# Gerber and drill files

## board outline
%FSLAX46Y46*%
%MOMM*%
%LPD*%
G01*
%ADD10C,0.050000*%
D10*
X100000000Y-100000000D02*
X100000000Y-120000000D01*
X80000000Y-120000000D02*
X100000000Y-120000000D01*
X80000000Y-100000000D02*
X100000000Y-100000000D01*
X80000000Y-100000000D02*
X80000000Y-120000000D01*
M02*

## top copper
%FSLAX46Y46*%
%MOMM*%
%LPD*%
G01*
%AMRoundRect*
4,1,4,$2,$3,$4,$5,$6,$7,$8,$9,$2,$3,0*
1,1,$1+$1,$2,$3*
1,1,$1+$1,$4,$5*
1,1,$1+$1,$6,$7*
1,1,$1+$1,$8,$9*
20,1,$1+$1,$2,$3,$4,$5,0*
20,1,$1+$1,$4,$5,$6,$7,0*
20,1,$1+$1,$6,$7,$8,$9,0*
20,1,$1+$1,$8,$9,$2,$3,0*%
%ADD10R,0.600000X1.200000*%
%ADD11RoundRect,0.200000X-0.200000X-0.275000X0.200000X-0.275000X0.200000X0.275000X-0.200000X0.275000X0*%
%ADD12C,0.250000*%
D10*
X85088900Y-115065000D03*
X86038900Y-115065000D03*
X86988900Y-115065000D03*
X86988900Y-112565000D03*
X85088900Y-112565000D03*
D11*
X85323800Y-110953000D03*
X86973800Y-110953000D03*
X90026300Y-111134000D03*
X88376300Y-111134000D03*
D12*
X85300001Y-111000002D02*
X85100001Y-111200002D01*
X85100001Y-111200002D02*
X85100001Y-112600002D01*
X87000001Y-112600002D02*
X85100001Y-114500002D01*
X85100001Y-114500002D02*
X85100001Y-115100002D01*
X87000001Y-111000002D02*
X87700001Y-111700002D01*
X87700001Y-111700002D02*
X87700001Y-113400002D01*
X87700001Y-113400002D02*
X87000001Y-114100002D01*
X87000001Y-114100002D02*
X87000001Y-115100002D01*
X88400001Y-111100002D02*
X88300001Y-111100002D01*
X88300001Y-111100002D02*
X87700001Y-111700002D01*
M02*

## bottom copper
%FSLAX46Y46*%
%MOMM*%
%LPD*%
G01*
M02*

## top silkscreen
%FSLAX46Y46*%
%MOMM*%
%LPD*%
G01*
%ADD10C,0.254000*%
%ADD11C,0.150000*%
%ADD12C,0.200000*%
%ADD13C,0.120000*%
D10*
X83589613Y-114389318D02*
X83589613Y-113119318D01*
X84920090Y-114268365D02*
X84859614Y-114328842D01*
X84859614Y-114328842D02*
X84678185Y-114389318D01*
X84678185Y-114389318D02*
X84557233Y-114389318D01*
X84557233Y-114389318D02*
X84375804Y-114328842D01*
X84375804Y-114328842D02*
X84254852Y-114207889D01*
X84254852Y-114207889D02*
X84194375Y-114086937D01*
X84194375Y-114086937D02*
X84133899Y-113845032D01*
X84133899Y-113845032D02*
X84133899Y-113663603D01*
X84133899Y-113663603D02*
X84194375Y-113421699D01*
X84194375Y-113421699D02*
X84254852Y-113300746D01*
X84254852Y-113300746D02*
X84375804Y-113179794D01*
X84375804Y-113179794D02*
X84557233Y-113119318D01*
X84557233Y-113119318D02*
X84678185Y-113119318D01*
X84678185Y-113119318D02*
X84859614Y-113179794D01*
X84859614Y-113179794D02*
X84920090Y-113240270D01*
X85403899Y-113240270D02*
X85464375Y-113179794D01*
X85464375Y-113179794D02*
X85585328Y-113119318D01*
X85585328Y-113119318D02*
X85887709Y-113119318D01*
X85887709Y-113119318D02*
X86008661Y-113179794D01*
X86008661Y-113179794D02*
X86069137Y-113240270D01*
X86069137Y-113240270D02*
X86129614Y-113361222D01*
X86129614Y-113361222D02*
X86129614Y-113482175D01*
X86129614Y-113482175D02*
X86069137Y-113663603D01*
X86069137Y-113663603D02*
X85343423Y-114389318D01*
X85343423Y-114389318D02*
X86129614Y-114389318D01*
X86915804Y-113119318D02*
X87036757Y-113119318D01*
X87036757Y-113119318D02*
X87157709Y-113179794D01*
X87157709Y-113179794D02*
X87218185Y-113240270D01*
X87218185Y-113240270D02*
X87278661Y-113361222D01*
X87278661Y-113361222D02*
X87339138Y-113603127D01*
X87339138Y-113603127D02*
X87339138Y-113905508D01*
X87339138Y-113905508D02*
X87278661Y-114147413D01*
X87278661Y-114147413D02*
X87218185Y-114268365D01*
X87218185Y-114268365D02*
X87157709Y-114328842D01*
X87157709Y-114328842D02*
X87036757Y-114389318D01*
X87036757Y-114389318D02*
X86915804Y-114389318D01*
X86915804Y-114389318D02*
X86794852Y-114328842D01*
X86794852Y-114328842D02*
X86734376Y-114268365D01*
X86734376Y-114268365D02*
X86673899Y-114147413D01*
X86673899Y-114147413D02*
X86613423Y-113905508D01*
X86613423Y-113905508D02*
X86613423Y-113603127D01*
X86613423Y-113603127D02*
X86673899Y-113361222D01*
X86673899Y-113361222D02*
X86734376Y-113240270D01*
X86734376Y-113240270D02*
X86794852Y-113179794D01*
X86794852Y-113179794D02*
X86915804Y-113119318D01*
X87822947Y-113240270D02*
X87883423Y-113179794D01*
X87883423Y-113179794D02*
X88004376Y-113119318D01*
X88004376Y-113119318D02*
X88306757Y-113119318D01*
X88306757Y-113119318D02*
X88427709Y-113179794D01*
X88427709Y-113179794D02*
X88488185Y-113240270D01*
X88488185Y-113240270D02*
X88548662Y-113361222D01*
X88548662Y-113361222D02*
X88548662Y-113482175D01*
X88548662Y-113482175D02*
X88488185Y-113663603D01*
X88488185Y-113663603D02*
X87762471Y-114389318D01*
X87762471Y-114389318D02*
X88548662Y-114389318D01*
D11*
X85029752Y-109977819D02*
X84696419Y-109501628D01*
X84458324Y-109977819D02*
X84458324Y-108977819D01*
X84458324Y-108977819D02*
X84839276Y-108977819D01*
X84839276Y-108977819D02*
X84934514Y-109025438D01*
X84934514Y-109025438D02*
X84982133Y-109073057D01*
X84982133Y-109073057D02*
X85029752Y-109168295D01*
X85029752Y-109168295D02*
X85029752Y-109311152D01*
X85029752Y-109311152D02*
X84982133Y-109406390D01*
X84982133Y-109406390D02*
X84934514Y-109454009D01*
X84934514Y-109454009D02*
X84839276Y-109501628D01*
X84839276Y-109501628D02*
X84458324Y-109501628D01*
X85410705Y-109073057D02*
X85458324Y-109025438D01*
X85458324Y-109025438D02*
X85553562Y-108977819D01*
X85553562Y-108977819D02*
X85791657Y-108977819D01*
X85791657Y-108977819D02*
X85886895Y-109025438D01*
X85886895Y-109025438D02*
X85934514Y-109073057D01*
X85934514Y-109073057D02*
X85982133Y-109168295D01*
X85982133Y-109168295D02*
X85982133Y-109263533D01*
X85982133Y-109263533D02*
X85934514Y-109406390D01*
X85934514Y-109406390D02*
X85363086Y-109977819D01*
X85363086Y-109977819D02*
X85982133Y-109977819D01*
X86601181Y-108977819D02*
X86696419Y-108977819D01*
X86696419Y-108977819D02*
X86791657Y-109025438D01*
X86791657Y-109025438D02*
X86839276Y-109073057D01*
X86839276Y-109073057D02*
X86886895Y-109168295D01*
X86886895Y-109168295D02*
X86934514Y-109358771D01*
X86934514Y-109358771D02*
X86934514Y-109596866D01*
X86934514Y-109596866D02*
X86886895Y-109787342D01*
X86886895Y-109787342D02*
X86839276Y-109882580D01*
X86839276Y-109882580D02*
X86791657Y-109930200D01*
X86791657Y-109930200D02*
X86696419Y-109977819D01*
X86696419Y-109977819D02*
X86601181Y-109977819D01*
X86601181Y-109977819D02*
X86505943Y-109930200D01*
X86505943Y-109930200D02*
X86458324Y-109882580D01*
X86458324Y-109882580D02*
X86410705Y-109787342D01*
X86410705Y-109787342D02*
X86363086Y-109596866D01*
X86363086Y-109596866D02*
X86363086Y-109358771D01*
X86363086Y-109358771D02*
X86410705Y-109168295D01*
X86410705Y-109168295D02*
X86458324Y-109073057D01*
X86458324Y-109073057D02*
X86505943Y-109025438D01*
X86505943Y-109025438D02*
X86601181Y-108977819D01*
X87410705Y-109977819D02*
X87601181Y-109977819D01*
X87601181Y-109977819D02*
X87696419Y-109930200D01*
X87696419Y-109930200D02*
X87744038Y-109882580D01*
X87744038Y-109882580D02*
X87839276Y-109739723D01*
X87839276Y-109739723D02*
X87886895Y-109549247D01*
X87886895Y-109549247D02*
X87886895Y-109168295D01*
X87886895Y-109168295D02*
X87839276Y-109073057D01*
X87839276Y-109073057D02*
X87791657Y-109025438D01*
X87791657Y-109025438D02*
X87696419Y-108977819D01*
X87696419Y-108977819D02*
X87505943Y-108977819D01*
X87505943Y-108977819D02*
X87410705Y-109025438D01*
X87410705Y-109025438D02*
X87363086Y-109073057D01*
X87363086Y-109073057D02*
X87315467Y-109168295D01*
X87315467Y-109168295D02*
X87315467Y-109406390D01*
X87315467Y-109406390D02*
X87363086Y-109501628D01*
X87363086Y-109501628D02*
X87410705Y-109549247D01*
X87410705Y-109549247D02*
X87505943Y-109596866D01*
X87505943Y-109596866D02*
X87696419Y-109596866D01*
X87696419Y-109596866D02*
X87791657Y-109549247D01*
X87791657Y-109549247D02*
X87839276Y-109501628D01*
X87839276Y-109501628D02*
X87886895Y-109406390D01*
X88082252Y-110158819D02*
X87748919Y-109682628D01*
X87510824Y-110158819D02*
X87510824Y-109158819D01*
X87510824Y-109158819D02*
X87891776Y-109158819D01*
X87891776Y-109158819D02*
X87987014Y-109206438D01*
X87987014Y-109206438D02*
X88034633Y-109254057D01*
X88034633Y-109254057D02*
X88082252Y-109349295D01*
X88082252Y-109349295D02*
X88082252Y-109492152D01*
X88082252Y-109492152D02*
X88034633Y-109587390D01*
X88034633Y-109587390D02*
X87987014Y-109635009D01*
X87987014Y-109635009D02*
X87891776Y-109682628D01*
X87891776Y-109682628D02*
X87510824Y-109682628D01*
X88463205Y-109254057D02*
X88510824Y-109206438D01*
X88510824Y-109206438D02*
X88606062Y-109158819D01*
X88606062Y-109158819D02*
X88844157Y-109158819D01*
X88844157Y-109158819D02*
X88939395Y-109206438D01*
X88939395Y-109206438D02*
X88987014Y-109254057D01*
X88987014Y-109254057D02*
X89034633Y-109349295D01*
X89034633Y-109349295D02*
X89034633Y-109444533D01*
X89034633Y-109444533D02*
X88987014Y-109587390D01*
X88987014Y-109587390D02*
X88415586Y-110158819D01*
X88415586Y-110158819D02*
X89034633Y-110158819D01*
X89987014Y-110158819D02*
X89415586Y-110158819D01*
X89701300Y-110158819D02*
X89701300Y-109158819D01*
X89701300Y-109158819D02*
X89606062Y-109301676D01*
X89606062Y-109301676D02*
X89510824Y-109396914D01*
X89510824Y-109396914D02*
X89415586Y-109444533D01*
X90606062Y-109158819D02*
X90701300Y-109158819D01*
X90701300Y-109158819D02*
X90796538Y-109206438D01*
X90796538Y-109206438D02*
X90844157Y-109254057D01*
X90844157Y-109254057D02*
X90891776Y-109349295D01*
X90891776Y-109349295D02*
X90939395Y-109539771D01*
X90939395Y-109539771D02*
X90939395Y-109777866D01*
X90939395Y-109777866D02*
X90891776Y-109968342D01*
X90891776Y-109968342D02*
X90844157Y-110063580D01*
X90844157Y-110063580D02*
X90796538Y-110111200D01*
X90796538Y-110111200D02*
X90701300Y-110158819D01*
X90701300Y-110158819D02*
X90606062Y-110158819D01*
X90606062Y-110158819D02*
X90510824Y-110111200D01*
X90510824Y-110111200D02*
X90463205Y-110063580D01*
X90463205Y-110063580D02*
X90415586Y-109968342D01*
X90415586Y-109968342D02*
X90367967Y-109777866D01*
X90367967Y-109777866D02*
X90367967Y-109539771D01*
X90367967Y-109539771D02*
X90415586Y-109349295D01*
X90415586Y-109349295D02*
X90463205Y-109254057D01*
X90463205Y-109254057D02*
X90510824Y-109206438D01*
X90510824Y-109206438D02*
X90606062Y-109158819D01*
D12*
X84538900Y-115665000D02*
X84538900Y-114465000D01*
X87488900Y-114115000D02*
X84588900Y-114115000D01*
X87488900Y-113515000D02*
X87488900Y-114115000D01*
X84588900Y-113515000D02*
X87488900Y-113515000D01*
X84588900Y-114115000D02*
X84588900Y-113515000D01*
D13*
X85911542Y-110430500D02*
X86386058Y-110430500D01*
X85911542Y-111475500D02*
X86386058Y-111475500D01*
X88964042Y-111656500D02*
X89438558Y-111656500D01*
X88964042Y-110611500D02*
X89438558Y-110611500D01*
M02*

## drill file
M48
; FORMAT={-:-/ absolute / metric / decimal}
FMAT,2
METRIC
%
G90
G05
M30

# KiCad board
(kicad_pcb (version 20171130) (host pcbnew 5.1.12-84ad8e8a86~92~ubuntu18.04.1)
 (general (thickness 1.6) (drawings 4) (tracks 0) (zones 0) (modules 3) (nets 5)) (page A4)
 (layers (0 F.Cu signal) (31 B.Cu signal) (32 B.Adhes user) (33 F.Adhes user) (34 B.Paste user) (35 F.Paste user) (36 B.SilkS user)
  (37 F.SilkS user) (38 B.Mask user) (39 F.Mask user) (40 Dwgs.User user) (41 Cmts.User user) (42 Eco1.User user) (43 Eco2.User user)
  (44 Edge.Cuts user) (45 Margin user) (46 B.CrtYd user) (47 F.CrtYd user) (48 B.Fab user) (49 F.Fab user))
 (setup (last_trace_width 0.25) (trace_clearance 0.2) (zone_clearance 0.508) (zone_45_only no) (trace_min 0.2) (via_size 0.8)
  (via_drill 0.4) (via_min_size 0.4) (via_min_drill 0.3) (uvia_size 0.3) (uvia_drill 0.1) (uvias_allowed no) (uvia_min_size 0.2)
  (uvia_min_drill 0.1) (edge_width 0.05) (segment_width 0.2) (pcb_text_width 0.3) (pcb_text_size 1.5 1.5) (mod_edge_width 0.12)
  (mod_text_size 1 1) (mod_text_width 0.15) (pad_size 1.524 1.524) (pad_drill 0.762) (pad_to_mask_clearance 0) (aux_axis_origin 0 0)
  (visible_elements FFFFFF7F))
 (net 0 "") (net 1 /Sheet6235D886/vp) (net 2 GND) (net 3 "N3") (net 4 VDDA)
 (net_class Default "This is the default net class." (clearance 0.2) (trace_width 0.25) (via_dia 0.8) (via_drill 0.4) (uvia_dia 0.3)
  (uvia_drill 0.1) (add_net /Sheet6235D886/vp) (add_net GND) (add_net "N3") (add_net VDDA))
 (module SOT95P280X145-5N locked (layer F.Cu) (at 86.038900 113.815000 90.000000)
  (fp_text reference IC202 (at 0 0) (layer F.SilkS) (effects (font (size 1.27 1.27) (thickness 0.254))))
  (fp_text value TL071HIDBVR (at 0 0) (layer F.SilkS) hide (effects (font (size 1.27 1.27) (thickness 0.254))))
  (fp_line (start -1.85 -1.5) (end -0.65 -1.5) (layer F.SilkS) (width 0.2))
  (fp_line (start -0.3 1.45) (end -0.3 -1.45) (layer F.SilkS) (width 0.2))
  (fp_line (start 0.3 1.45) (end -0.3 1.45) (layer F.SilkS) (width 0.2))
  (fp_line (start 0.3 -1.45) (end 0.3 1.45) (layer F.SilkS) (width 0.2))
  (fp_line (start -0.3 -1.45) (end 0.3 -1.45) (layer F.SilkS) (width 0.2))
  (pad 1 smd rect (at -1.25 -0.95 180.000000) (size 0.6 1.2) (layers F.Cu F.Mask F.Paste) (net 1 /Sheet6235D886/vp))
  (pad 2 smd rect (at -1.25 0 180.000000) (size 0.6 1.2) (layers F.Cu F.Mask F.Paste) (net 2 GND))
  (pad 3 smd rect (at -1.25 0.95 180.000000) (size 0.6 1.2) (layers F.Cu F.Mask F.Paste) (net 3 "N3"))
  (pad 4 smd rect (at 1.25 0.95 180.000000) (size 0.6 1.2) (layers F.Cu F.Mask F.Paste) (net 1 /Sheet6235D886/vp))
  (pad 5 smd rect (at 1.25 -0.95 180.000000) (size 0.6 1.2) (layers F.Cu F.Mask F.Paste) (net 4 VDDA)))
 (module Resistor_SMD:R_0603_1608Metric (layer F.Cu) (at 86.148800 110.953000)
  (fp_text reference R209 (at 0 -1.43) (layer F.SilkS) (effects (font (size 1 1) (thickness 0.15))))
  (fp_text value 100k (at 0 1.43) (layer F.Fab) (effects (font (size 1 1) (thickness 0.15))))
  (fp_line (start -0.237258 -0.5225) (end 0.237258 -0.5225) (layer F.SilkS) (width 0.12))
  (fp_line (start -0.237258 0.5225) (end 0.237258 0.5225) (layer F.SilkS) (width 0.12))
  (pad 1 smd roundrect (at -0.825 0) (size 0.8 0.95) (layers F.Cu F.Mask F.Paste) (roundrect_rratio 0.25) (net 4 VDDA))
  (pad 2 smd roundrect (at 0.825 0) (size 0.8 0.95) (layers F.Cu F.Mask F.Paste) (roundrect_rratio 0.25) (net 3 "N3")))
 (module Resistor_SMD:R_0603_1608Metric (layer F.Cu) (at 89.201300 111.134000)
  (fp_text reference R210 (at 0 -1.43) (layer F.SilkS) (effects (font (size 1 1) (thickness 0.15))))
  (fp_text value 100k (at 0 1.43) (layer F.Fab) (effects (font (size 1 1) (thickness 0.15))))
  (fp_line (start -0.237258 0.5225) (end 0.237258 0.5225) (layer F.SilkS) (width 0.12))
  (fp_line (start -0.237258 -0.5225) (end 0.237258 -0.5225) (layer F.SilkS) (width 0.12))
  (pad 2 smd roundrect (at 0.825 0) (size 0.8 0.95) (layers F.Cu F.Mask F.Paste) (roundrect_rratio 0.25) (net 2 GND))
  (pad 1 smd roundrect (at -0.825 0) (size 0.8 0.95) (layers F.Cu F.Mask F.Paste) (roundrect_rratio 0.25) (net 3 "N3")))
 (gr_line (start 100 100) (end 100 120) (layer Edge.Cuts) (width 0.05))
 (gr_line (start 80 120) (end 100 120) (layer Edge.Cuts) (width 0.05))
 (gr_line (start 80 100) (end 100 100) (layer Edge.Cuts) (width 0.05))
 (gr_line (start 80 100) (end 80 120) (layer Edge.Cuts) (width 0.05))
 (segment (start 85.300001 111.000002) (end 85.100001 111.200002) (width 0.250000) (layer F.Cu) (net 4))
 (segment (start 85.100001 111.200002) (end 85.100001 112.600002) (width 0.250000) (layer F.Cu) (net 4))
 (segment (start 87.000001 112.600002) (end 85.100001 114.500002) (width 0.250000) (layer F.Cu) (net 1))
 (segment (start 85.100001 114.500002) (end 85.100001 115.100002) (width 0.250000) (layer F.Cu) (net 1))
 (segment (start 87.000001 111.000002) (end 87.700001 111.700002) (width 0.250000) (layer F.Cu) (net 3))
 (segment (start 87.700001 111.700002) (end 87.700001 113.400002) (width 0.250000) (layer F.Cu) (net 3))
 (segment (start 87.700001 113.400002) (end 87.000001 114.100002) (width 0.250000) (layer F.Cu) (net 3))
 (segment (start 87.000001 114.100002) (end 87.000001 115.100002) (width 0.250000) (layer F.Cu) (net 3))
 (segment (start 88.400001 111.100002) (end 88.300001 111.100002) (width 0.250000) (layer F.Cu) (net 3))
 (segment (start 88.300001 111.100002) (end 87.700001 111.700002) (width 0.250000) (layer F.Cu) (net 3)))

